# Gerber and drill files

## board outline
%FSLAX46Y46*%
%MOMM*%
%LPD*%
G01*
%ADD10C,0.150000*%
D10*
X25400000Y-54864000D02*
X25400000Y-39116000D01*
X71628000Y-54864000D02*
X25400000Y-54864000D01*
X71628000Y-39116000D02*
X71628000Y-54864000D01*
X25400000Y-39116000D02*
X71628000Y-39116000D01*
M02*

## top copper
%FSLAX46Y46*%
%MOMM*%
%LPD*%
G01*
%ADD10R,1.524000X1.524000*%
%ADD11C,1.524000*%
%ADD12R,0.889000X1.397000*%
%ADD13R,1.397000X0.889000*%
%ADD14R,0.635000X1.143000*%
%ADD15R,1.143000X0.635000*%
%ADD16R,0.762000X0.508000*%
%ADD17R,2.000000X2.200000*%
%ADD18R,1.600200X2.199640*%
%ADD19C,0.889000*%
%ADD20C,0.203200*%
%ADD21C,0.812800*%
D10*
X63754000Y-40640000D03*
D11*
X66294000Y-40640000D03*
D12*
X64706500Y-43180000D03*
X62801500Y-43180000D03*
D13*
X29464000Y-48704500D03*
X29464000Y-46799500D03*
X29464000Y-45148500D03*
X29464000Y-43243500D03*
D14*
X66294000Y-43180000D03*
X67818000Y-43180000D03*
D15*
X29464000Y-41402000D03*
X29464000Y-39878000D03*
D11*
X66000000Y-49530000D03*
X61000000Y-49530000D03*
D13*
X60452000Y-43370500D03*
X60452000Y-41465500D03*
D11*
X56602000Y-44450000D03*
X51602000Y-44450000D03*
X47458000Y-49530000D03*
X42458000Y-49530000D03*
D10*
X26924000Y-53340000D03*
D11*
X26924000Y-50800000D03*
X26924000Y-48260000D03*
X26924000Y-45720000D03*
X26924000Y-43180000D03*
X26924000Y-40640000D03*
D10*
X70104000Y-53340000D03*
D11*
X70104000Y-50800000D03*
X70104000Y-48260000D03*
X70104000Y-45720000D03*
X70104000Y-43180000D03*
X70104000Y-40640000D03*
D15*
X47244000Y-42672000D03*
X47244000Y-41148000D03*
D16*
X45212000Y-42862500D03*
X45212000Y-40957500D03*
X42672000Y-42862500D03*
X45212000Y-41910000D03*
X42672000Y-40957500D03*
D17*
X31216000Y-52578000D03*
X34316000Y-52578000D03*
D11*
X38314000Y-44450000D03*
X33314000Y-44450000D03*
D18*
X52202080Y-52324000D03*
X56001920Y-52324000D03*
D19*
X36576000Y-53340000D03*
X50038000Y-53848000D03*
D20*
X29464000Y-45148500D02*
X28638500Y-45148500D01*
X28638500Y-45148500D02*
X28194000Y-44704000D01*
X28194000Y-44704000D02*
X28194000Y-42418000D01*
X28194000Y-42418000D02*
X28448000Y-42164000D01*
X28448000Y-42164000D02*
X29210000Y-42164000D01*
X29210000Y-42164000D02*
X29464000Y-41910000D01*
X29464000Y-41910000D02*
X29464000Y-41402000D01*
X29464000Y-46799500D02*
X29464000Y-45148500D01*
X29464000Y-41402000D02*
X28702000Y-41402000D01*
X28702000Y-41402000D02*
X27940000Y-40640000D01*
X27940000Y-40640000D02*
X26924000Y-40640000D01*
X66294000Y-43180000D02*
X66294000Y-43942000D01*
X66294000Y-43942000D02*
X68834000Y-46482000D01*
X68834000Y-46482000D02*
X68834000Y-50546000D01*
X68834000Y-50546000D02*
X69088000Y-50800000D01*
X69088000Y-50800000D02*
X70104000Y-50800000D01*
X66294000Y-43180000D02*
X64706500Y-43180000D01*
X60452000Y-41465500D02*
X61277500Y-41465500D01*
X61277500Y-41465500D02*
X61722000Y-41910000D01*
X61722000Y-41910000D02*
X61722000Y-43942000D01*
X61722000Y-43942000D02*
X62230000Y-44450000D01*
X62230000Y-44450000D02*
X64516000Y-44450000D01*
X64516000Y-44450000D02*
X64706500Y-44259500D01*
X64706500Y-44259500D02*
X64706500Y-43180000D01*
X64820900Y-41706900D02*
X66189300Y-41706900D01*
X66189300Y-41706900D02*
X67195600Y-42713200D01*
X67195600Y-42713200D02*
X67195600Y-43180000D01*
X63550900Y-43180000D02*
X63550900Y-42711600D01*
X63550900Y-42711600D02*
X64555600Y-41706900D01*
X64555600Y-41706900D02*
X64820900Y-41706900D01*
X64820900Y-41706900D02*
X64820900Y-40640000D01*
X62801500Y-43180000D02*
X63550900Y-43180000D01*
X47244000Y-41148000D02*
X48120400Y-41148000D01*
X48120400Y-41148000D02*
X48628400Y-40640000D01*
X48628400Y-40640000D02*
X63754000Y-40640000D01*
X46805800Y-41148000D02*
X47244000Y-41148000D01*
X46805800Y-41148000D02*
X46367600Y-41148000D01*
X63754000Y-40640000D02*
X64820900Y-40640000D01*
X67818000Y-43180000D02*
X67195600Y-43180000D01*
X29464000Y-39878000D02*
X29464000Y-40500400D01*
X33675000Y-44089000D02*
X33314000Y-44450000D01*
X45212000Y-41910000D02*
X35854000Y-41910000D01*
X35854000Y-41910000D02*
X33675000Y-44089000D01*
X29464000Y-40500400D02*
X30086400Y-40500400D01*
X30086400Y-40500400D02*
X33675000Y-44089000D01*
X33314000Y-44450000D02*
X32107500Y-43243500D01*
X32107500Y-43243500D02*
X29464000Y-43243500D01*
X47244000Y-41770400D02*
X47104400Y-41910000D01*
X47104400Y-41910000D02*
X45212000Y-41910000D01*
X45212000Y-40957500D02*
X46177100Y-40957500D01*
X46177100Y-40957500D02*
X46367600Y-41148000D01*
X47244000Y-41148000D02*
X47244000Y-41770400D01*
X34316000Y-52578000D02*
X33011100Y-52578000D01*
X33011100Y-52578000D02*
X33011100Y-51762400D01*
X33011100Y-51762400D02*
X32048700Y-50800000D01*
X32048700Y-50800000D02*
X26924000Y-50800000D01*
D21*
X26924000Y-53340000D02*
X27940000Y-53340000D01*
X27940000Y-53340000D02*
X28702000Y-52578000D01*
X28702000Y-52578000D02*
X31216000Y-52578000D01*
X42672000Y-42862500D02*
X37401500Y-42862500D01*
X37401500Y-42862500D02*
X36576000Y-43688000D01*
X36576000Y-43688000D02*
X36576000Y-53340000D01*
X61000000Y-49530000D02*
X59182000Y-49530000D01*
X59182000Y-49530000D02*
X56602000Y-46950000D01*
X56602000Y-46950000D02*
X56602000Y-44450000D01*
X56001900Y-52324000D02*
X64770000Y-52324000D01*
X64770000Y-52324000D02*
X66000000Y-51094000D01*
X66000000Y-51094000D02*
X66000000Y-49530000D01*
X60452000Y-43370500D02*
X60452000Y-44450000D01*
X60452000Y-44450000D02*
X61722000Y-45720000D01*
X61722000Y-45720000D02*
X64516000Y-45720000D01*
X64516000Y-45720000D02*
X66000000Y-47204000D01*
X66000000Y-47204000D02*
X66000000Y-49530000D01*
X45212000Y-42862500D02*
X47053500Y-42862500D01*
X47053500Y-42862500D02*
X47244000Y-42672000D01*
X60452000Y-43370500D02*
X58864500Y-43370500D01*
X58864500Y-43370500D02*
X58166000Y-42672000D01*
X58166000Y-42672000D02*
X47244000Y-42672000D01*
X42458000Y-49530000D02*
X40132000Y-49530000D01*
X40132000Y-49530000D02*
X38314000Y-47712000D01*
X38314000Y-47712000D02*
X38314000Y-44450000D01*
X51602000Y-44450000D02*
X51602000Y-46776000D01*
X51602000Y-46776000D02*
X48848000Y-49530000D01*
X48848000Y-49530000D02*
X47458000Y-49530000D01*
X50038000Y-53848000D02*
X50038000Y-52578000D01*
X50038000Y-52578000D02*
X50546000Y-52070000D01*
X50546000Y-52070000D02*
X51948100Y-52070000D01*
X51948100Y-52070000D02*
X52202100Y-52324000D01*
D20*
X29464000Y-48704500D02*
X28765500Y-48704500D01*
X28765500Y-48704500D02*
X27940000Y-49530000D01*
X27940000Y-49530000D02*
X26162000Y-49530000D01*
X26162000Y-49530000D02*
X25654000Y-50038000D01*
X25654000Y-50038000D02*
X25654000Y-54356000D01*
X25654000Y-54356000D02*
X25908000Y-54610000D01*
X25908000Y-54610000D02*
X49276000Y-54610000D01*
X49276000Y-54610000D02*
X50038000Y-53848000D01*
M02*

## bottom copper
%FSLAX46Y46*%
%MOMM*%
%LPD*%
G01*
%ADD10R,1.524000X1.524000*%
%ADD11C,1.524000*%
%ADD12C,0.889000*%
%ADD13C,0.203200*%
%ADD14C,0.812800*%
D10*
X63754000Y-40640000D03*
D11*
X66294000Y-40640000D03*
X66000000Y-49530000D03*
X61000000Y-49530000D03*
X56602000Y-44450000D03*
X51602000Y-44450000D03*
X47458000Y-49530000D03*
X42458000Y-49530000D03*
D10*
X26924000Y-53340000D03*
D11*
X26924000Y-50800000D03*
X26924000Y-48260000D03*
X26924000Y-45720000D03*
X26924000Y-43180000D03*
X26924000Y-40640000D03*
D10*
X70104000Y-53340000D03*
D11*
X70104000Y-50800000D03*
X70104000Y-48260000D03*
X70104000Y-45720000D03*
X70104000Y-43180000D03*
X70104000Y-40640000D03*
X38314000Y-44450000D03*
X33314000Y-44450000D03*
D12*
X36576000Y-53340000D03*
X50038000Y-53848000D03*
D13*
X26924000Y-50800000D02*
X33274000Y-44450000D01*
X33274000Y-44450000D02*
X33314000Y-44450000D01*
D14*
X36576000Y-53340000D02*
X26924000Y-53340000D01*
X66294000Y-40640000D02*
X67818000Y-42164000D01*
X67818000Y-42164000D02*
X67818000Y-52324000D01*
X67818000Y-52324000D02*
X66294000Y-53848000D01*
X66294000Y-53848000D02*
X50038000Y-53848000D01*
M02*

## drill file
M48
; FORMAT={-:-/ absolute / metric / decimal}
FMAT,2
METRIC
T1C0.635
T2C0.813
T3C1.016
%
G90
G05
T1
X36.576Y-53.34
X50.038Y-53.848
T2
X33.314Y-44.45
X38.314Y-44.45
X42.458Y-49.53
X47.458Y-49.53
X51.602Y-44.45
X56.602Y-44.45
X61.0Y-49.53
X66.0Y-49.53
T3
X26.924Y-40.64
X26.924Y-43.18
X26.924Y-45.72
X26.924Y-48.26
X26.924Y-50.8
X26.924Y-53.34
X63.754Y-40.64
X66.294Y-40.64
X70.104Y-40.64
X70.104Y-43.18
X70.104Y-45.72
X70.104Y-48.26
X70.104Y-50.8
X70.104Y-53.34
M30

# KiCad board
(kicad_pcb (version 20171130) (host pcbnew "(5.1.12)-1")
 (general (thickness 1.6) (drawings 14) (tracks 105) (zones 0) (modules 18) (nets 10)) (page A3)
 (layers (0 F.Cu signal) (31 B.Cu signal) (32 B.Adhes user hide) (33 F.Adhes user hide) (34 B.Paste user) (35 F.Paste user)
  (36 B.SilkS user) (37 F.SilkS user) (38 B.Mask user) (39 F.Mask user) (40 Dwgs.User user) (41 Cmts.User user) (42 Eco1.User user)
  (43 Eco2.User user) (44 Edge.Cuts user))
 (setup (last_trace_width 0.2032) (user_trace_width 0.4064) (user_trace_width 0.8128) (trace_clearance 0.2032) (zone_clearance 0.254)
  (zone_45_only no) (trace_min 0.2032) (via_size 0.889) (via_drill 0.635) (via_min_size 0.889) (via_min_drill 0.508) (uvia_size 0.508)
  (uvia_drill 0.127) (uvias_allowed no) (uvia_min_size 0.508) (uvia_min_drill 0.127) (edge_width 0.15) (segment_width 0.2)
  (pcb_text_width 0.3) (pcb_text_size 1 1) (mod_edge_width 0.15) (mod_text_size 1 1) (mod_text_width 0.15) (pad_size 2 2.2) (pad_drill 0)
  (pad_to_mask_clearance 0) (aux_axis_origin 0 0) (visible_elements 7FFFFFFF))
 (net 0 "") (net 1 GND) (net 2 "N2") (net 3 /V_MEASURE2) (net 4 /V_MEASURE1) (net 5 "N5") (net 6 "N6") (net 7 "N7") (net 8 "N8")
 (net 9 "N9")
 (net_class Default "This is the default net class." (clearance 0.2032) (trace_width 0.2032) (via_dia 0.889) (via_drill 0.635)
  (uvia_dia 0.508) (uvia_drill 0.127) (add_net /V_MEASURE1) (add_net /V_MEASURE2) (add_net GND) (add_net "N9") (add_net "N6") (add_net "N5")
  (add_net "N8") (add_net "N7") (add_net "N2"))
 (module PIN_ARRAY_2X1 (layer F.Cu) (at 65.024 40.64)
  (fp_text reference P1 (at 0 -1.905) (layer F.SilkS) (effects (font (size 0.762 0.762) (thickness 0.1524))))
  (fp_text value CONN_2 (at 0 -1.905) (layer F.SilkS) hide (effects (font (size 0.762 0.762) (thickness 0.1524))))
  (pad 1 thru_hole rect (at -1.27 0) (size 1.524 1.524) (drill 1.016) (layers *.Cu *.Mask F.SilkS) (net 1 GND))
  (pad 2 thru_hole circle (at 1.27 0) (size 1.524 1.524) (drill 1.016) (layers *.Cu *.Mask F.SilkS) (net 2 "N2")))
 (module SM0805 (layer F.Cu) (at 63.754 43.18 180)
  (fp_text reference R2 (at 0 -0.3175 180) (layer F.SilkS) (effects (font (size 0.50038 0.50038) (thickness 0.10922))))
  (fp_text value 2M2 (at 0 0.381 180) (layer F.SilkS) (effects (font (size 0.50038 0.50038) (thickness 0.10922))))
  (pad 1 smd rect (at -0.9525 0 180) (size 0.889 1.397) (layers F.Cu F.Paste F.Mask) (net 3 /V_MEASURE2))
  (pad 2 smd rect (at 0.9525 0 180) (size 0.889 1.397) (layers F.Cu F.Paste F.Mask) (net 1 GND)))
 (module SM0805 (layer F.Cu) (at 29.464 47.752 90)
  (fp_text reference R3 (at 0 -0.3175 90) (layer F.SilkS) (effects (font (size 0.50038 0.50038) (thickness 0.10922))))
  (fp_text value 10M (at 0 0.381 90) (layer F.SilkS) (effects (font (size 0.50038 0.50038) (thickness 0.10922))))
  (pad 1 smd rect (at -0.9525 0 90) (size 0.889 1.397) (layers F.Cu F.Paste F.Mask) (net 2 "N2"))
  (pad 2 smd rect (at 0.9525 0 90) (size 0.889 1.397) (layers F.Cu F.Paste F.Mask) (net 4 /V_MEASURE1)))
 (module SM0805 (layer F.Cu) (at 29.464 44.196 90)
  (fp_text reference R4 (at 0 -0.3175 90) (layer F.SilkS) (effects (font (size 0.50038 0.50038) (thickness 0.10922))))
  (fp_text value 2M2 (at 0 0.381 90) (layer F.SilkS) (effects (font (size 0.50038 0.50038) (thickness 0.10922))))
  (pad 1 smd rect (at -0.9525 0 90) (size 0.889 1.397) (layers F.Cu F.Paste F.Mask) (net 4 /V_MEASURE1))
  (pad 2 smd rect (at 0.9525 0 90) (size 0.889 1.397) (layers F.Cu F.Paste F.Mask) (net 1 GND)))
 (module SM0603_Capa (layer F.Cu) (at 67.056 43.18)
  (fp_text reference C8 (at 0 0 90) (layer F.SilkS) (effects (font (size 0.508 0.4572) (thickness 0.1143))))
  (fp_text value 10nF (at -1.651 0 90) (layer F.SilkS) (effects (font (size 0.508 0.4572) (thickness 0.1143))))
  (pad 1 smd rect (at -0.762 0) (size 0.635 1.143) (layers F.Cu F.Paste F.Mask) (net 3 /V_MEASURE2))
  (pad 2 smd rect (at 0.762 0) (size 0.635 1.143) (layers F.Cu F.Paste F.Mask) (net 1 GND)))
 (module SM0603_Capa (layer F.Cu) (at 29.464 40.64 90)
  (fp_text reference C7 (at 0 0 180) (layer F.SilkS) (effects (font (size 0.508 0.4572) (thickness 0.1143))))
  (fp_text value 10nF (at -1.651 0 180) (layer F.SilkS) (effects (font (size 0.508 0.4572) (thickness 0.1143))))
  (pad 1 smd rect (at -0.762 0 90) (size 0.635 1.143) (layers F.Cu F.Paste F.Mask) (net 4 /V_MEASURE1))
  (pad 2 smd rect (at 0.762 0 90) (size 0.635 1.143) (layers F.Cu F.Paste F.Mask) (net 1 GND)))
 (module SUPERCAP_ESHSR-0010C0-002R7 (layer F.Cu) (at 63.5 49.53 180)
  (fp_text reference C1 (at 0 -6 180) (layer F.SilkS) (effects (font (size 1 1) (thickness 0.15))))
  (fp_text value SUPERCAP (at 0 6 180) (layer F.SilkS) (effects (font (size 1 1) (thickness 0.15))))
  (pad 1 thru_hole circle (at -2.5 0 180) (size 1.524 1.524) (drill 0.8128) (layers *.Cu *.Mask F.SilkS) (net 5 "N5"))
  (pad 2 thru_hole circle (at 2.5 0 180) (size 1.524 1.524) (drill 0.8128) (layers *.Cu *.Mask F.SilkS) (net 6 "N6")))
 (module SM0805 (layer F.Cu) (at 60.452 42.418 90)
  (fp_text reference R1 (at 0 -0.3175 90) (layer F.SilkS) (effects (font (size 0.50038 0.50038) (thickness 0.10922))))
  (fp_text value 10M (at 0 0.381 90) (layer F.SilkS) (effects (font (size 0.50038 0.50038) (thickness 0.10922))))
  (pad 1 smd rect (at -0.9525 0 90) (size 0.889 1.397) (layers F.Cu F.Paste F.Mask) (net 5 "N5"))
  (pad 2 smd rect (at 0.9525 0 90) (size 0.889 1.397) (layers F.Cu F.Paste F.Mask) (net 3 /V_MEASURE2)))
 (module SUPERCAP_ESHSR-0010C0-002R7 (layer F.Cu) (at 54.102 44.45 180)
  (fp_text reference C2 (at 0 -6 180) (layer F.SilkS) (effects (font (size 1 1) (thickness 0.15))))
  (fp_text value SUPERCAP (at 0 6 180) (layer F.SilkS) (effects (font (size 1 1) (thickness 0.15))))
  (pad 1 thru_hole circle (at -2.5 0 180) (size 1.524 1.524) (drill 0.8128) (layers *.Cu *.Mask F.SilkS) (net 6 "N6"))
  (pad 2 thru_hole circle (at 2.5 0 180) (size 1.524 1.524) (drill 0.8128) (layers *.Cu *.Mask F.SilkS) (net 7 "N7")))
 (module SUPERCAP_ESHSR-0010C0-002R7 (layer F.Cu) (at 44.958 49.53 180)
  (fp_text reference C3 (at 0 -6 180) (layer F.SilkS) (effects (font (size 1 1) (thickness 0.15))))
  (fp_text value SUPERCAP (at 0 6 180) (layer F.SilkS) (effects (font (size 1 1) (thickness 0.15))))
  (pad 1 thru_hole circle (at -2.5 0 180) (size 1.524 1.524) (drill 0.8128) (layers *.Cu *.Mask F.SilkS) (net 7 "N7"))
  (pad 2 thru_hole circle (at 2.5 0 180) (size 1.524 1.524) (drill 0.8128) (layers *.Cu *.Mask F.SilkS) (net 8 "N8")))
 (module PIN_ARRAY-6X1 (layer F.Cu) (at 26.924 46.99 90)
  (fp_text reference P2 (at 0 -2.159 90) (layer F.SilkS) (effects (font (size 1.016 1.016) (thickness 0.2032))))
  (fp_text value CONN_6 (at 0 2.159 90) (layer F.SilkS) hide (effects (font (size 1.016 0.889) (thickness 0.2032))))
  (pad 1 thru_hole rect (at -6.35 0 90) (size 1.524 1.524) (drill 1.016) (layers *.Cu *.Mask F.SilkS) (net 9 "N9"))
  (pad 2 thru_hole circle (at -3.81 0 90) (size 1.524 1.524) (drill 1.016) (layers *.Cu *.Mask F.SilkS) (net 1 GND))
  (pad 3 thru_hole circle (at -1.27 0 90) (size 1.524 1.524) (drill 1.016) (layers *.Cu *.Mask F.SilkS))
  (pad 4 thru_hole circle (at 1.27 0 90) (size 1.524 1.524) (drill 1.016) (layers *.Cu *.Mask F.SilkS))
  (pad 5 thru_hole circle (at 3.81 0 90) (size 1.524 1.524) (drill 1.016) (layers *.Cu *.Mask F.SilkS))
  (pad 6 thru_hole circle (at 6.35 0 90) (size 1.524 1.524) (drill 1.016) (layers *.Cu *.Mask F.SilkS) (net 4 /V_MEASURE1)))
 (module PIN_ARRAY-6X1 (layer F.Cu) (at 70.104 46.99 90)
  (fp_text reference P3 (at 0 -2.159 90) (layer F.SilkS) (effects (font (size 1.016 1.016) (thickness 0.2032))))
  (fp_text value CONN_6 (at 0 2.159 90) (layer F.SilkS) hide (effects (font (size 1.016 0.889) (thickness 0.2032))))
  (pad 1 thru_hole rect (at -6.35 0 90) (size 1.524 1.524) (drill 1.016) (layers *.Cu *.Mask F.SilkS))
  (pad 2 thru_hole circle (at -3.81 0 90) (size 1.524 1.524) (drill 1.016) (layers *.Cu *.Mask F.SilkS) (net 3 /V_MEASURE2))
  (pad 3 thru_hole circle (at -1.27 0 90) (size 1.524 1.524) (drill 1.016) (layers *.Cu *.Mask F.SilkS))
  (pad 4 thru_hole circle (at 1.27 0 90) (size 1.524 1.524) (drill 1.016) (layers *.Cu *.Mask F.SilkS))
  (pad 5 thru_hole circle (at 3.81 0 90) (size 1.524 1.524) (drill 1.016) (layers *.Cu *.Mask F.SilkS))
  (pad 6 thru_hole circle (at 6.35 0 90) (size 1.524 1.524) (drill 1.016) (layers *.Cu *.Mask F.SilkS)))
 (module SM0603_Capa (layer F.Cu) (at 47.244 41.91 90)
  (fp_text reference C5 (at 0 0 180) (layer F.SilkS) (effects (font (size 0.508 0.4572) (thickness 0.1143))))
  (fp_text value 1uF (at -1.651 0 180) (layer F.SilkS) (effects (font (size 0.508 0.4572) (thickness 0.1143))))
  (pad 1 smd rect (at -0.762 0 90) (size 0.635 1.143) (layers F.Cu F.Paste F.Mask) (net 5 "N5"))
  (pad 2 smd rect (at 0.762 0 90) (size 0.635 1.143) (layers F.Cu F.Paste F.Mask) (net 1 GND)))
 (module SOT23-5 (layer F.Cu) (at 43.942 41.91 90)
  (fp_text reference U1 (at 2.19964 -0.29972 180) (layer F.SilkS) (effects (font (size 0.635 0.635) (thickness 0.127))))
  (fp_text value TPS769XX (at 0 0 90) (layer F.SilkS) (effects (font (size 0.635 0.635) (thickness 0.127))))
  (pad 1 smd rect (at -0.9525 1.27 90) (size 0.508 0.762) (layers F.Cu F.Paste F.Mask) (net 5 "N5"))
  (pad 3 smd rect (at 0.9525 1.27 90) (size 0.508 0.762) (layers F.Cu F.Paste F.Mask) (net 1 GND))
  (pad 5 smd rect (at -0.9525 -1.27 90) (size 0.508 0.762) (layers F.Cu F.Paste F.Mask) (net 9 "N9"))
  (pad 2 smd rect (at 0 1.27 90) (size 0.508 0.762) (layers F.Cu F.Paste F.Mask) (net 1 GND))
  (pad 4 smd rect (at 0.9525 -1.27 90) (size 0.508 0.762) (layers F.Cu F.Paste F.Mask)))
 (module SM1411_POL (layer F.Cu) (at 32.766 52.578)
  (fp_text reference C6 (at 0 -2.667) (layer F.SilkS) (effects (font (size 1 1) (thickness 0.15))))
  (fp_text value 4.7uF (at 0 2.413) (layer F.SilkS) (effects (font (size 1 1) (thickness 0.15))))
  (pad 1 smd rect (at -1.55 0) (size 2 2.2) (layers F.Cu F.Paste F.Mask) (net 9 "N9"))
  (pad 2 smd rect (at 1.55 0) (size 2 2.2) (layers F.Cu F.Paste F.Mask) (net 1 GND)))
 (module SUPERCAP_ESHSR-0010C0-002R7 (layer F.Cu) (at 35.814 44.45 180)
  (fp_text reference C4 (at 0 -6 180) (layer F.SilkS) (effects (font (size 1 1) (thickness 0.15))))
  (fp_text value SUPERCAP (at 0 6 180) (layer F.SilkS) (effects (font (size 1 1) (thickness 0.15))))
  (pad 1 thru_hole circle (at -2.5 0 180) (size 1.524 1.524) (drill 0.8128) (layers *.Cu *.Mask F.SilkS) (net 8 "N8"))
  (pad 2 thru_hole circle (at 2.5 0 180) (size 1.524 1.524) (drill 0.8128) (layers *.Cu *.Mask F.SilkS) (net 1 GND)))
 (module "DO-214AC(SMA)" (layer F.Cu) (at 54.102 52.324)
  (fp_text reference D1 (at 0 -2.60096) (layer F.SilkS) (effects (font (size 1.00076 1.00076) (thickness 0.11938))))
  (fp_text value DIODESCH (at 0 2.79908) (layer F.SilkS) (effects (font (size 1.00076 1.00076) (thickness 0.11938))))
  (pad 1 smd rect (at -1.89992 0) (size 1.6002 2.19964) (layers F.Cu F.Paste F.Mask) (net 2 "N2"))
  (pad 2 smd rect (at 1.89992 0) (size 1.6002 2.19964) (layers F.Cu F.Paste F.Mask) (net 5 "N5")))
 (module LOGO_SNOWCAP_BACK (layer B.Cu) (at 48.768 46.482)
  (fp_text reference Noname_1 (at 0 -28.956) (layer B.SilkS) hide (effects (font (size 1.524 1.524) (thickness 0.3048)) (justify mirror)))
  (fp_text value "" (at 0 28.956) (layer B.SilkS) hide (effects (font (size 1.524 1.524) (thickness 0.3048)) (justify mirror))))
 (gr_line (start 25.4 54.864) (end 25.4 39.116) (angle 90) (layer Edge.Cuts) (width 0.15))
 (gr_line (start 71.628 54.864) (end 25.4 54.864) (angle 90) (layer Edge.Cuts) (width 0.15))
 (gr_line (start 71.628 39.116) (end 71.628 54.864) (angle 90) (layer Edge.Cuts) (width 0.15))
 (gr_line (start 25.4 39.116) (end 71.628 39.116) (angle 90) (layer Edge.Cuts) (width 0.15))
 (segment (start 29.464 45.1485) (end 28.6385 45.1485) (width 0.2032) (layer F.Cu) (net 4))
 (segment (start 28.6385 45.1485) (end 28.194 44.704) (width 0.2032) (layer F.Cu) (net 4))
 (segment (start 28.194 44.704) (end 28.194 42.418) (width 0.2032) (layer F.Cu) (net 4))
 (segment (start 28.194 42.418) (end 28.448 42.164) (width 0.2032) (layer F.Cu) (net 4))
 (segment (start 28.448 42.164) (end 29.21 42.164) (width 0.2032) (layer F.Cu) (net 4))
 (segment (start 29.21 42.164) (end 29.464 41.91) (width 0.2032) (layer F.Cu) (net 4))
 (segment (start 29.464 41.91) (end 29.464 41.402) (width 0.2032) (layer F.Cu) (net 4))
 (segment (start 29.464 46.7995) (end 29.464 45.1485) (width 0.2032) (layer F.Cu) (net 4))
 (segment (start 29.464 41.402) (end 28.702 41.402) (width 0.2032) (layer F.Cu) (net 4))
 (segment (start 28.702 41.402) (end 27.94 40.64) (width 0.2032) (layer F.Cu) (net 4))
 (segment (start 27.94 40.64) (end 26.924 40.64) (width 0.2032) (layer F.Cu) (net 4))
 (segment (start 66.294 43.18) (end 66.294 43.942) (width 0.2032) (layer F.Cu) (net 3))
 (segment (start 66.294 43.942) (end 68.834 46.482) (width 0.2032) (layer F.Cu) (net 3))
 (segment (start 68.834 46.482) (end 68.834 50.546) (width 0.2032) (layer F.Cu) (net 3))
 (segment (start 68.834 50.546) (end 69.088 50.8) (width 0.2032) (layer F.Cu) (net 3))
 (segment (start 69.088 50.8) (end 70.104 50.8) (width 0.2032) (layer F.Cu) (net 3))
 (segment (start 66.294 43.18) (end 64.7065 43.18) (width 0.2032) (layer F.Cu) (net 3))
 (segment (start 60.452 41.4655) (end 61.2775 41.4655) (width 0.2032) (layer F.Cu) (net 3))
 (segment (start 61.2775 41.4655) (end 61.722 41.91) (width 0.2032) (layer F.Cu) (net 3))
 (segment (start 61.722 41.91) (end 61.722 43.942) (width 0.2032) (layer F.Cu) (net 3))
 (segment (start 61.722 43.942) (end 62.23 44.45) (width 0.2032) (layer F.Cu) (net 3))
 (segment (start 62.23 44.45) (end 64.516 44.45) (width 0.2032) (layer F.Cu) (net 3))
 (segment (start 64.516 44.45) (end 64.7065 44.2595) (width 0.2032) (layer F.Cu) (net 3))
 (segment (start 64.7065 44.2595) (end 64.7065 43.18) (width 0.2032) (layer F.Cu) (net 3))
 (segment (start 64.8209 41.7069) (end 66.1893 41.7069) (width 0.2032) (layer F.Cu) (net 1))
 (segment (start 66.1893 41.7069) (end 67.1956 42.7132) (width 0.2032) (layer F.Cu) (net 1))
 (segment (start 67.1956 42.7132) (end 67.1956 43.18) (width 0.2032) (layer F.Cu) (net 1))
 (segment (start 63.5509 43.18) (end 63.5509 42.7116) (width 0.2032) (layer F.Cu) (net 1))
 (segment (start 63.5509 42.7116) (end 64.5556 41.7069) (width 0.2032) (layer F.Cu) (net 1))
 (segment (start 64.5556 41.7069) (end 64.8209 41.7069) (width 0.2032) (layer F.Cu) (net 1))
 (segment (start 64.8209 41.7069) (end 64.8209 40.64) (width 0.2032) (layer F.Cu) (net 1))
 (segment (start 62.8015 43.18) (end 63.5509 43.18) (width 0.2032) (layer F.Cu) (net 1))
 (segment (start 47.244 41.148) (end 48.1204 41.148) (width 0.2032) (layer F.Cu) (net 1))
 (segment (start 48.1204 41.148) (end 48.6284 40.64) (width 0.2032) (layer F.Cu) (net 1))
 (segment (start 48.6284 40.64) (end 63.754 40.64) (width 0.2032) (layer F.Cu) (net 1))
 (segment (start 46.8058 41.148) (end 47.244 41.148) (width 0.2032) (layer F.Cu) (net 1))
 (segment (start 46.8058 41.148) (end 46.3676 41.148) (width 0.2032) (layer F.Cu) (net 1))
 (segment (start 63.754 40.64) (end 64.8209 40.64) (width 0.2032) (layer F.Cu) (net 1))
 (segment (start 67.818 43.18) (end 67.1956 43.18) (width 0.2032) (layer F.Cu) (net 1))
 (segment (start 29.464 39.878) (end 29.464 40.5004) (width 0.2032) (layer F.Cu) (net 1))
 (segment (start 33.675 44.089) (end 33.314 44.45) (width 0.2032) (layer F.Cu) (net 1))
 (segment (start 45.212 41.91) (end 35.854 41.91) (width 0.2032) (layer F.Cu) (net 1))
 (segment (start 35.854 41.91) (end 33.675 44.089) (width 0.2032) (layer F.Cu) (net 1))
 (segment (start 29.464 40.5004) (end 30.0864 40.5004) (width 0.2032) (layer F.Cu) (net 1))
 (segment (start 30.0864 40.5004) (end 33.675 44.089) (width 0.2032) (layer F.Cu) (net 1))
 (segment (start 33.314 44.45) (end 32.1075 43.2435) (width 0.2032) (layer F.Cu) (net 1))
 (segment (start 32.1075 43.2435) (end 29.464 43.2435) (width 0.2032) (layer F.Cu) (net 1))
 (segment (start 47.244 41.7704) (end 47.1044 41.91) (width 0.2032) (layer F.Cu) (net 1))
 (segment (start 47.1044 41.91) (end 45.212 41.91) (width 0.2032) (layer F.Cu) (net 1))
 (segment (start 26.924 50.8) (end 33.274 44.45) (width 0.2032) (layer B.Cu) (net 1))
 (segment (start 33.274 44.45) (end 33.314 44.45) (width 0.2032) (layer B.Cu) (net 1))
 (segment (start 45.212 40.9575) (end 46.1771 40.9575) (width 0.2032) (layer F.Cu) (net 1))
 (segment (start 46.1771 40.9575) (end 46.3676 41.148) (width 0.2032) (layer F.Cu) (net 1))
 (segment (start 47.244 41.148) (end 47.244 41.7704) (width 0.2032) (layer F.Cu) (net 1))
 (segment (start 34.316 52.578) (end 33.0111 52.578) (width 0.2032) (layer F.Cu) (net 1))
 (segment (start 33.0111 52.578) (end 33.0111 51.7624) (width 0.2032) (layer F.Cu) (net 1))
 (segment (start 33.0111 51.7624) (end 32.0487 50.8) (width 0.2032) (layer F.Cu) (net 1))
 (segment (start 32.0487 50.8) (end 26.924 50.8) (width 0.2032) (layer F.Cu) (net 1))
 (segment (start 26.924 53.34) (end 27.94 53.34) (width 0.8128) (layer F.Cu) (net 9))
 (segment (start 27.94 53.34) (end 28.702 52.578) (width 0.8128) (layer F.Cu) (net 9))
 (segment (start 28.702 52.578) (end 31.216 52.578) (width 0.8128) (layer F.Cu) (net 9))
 (segment (start 42.672 42.8625) (end 37.4015 42.8625) (width 0.8128) (layer F.Cu) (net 9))
 (segment (start 37.4015 42.8625) (end 36.576 43.688) (width 0.8128) (layer F.Cu) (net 9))
 (segment (start 36.576 43.688) (end 36.576 53.34) (width 0.8128) (layer F.Cu) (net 9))
 (segment (start 36.576 53.34) (end 26.924 53.34) (width 0.8128) (layer B.Cu) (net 9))
 (via (at 36.576 53.34) (size 0.889) (layers F.Cu B.Cu) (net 9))
 (segment (start 61 49.53) (end 59.182 49.53) (width 0.8128) (layer F.Cu) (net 6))
 (segment (start 59.182 49.53) (end 56.602 46.95) (width 0.8128) (layer F.Cu) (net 6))
 (segment (start 56.602 46.95) (end 56.602 44.45) (width 0.8128) (layer F.Cu) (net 6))
 (segment (start 56.0019 52.324) (end 64.77 52.324) (width 0.8128) (layer F.Cu) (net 5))
 (segment (start 64.77 52.324) (end 66 51.094) (width 0.8128) (layer F.Cu) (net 5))
 (segment (start 66 51.094) (end 66 49.53) (width 0.8128) (layer F.Cu) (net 5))
 (segment (start 60.452 43.3705) (end 60.452 44.45) (width 0.8128) (layer F.Cu) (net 5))
 (segment (start 60.452 44.45) (end 61.722 45.72) (width 0.8128) (layer F.Cu) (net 5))
 (segment (start 61.722 45.72) (end 64.516 45.72) (width 0.8128) (layer F.Cu) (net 5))
 (segment (start 64.516 45.72) (end 66 47.204) (width 0.8128) (layer F.Cu) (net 5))
 (segment (start 66 47.204) (end 66 49.53) (width 0.8128) (layer F.Cu) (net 5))
 (segment (start 45.212 42.8625) (end 47.0535 42.8625) (width 0.8128) (layer F.Cu) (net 5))
 (segment (start 47.0535 42.8625) (end 47.244 42.672) (width 0.8128) (layer F.Cu) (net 5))
 (segment (start 60.452 43.3705) (end 58.8645 43.3705) (width 0.8128) (layer F.Cu) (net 5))
 (segment (start 58.8645 43.3705) (end 58.166 42.672) (width 0.8128) (layer F.Cu) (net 5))
 (segment (start 58.166 42.672) (end 47.244 42.672) (width 0.8128) (layer F.Cu) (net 5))
 (segment (start 42.458 49.53) (end 40.132 49.53) (width 0.8128) (layer F.Cu) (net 8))
 (segment (start 40.132 49.53) (end 38.314 47.712) (width 0.8128) (layer F.Cu) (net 8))
 (segment (start 38.314 47.712) (end 38.314 44.45) (width 0.8128) (layer F.Cu) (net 8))
 (segment (start 51.602 44.45) (end 51.602 46.776) (width 0.8128) (layer F.Cu) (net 7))
 (segment (start 51.602 46.776) (end 48.848 49.53) (width 0.8128) (layer F.Cu) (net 7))
 (segment (start 48.848 49.53) (end 47.458 49.53) (width 0.8128) (layer F.Cu) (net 7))
 (segment (start 66.294 40.64) (end 67.818 42.164) (width 0.8128) (layer B.Cu) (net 2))
 (segment (start 67.818 42.164) (end 67.818 52.324) (width 0.8128) (layer B.Cu) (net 2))
 (segment (start 67.818 52.324) (end 66.294 53.848) (width 0.8128) (layer B.Cu) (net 2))
 (segment (start 66.294 53.848) (end 50.038 53.848) (width 0.8128) (layer B.Cu) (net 2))
 (segment (start 50.038 53.848) (end 50.038 52.578) (width 0.8128) (layer F.Cu) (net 2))
 (segment (start 50.038 52.578) (end 50.546 52.07) (width 0.8128) (layer F.Cu) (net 2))
 (segment (start 50.546 52.07) (end 51.9481 52.07) (width 0.8128) (layer F.Cu) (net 2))
 (segment (start 51.9481 52.07) (end 52.2021 52.324) (width 0.8128) (layer F.Cu) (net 2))
 (segment (start 29.464 48.7045) (end 28.7655 48.7045) (width 0.2032) (layer F.Cu) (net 2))
 (segment (start 28.7655 48.7045) (end 27.94 49.53) (width 0.2032) (layer F.Cu) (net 2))
 (segment (start 27.94 49.53) (end 26.162 49.53) (width 0.2032) (layer F.Cu) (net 2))
 (segment (start 26.162 49.53) (end 25.654 50.038) (width 0.2032) (layer F.Cu) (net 2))
 (segment (start 25.654 50.038) (end 25.654 54.356) (width 0.2032) (layer F.Cu) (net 2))
 (segment (start 25.654 54.356) (end 25.908 54.61) (width 0.2032) (layer F.Cu) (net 2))
 (segment (start 25.908 54.61) (end 49.276 54.61) (width 0.2032) (layer F.Cu) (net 2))
 (segment (start 49.276 54.61) (end 50.038 53.848) (width 0.2032) (layer F.Cu) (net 2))
 (via (at 50.038 53.848) (size 0.889) (layers F.Cu B.Cu) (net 2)))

